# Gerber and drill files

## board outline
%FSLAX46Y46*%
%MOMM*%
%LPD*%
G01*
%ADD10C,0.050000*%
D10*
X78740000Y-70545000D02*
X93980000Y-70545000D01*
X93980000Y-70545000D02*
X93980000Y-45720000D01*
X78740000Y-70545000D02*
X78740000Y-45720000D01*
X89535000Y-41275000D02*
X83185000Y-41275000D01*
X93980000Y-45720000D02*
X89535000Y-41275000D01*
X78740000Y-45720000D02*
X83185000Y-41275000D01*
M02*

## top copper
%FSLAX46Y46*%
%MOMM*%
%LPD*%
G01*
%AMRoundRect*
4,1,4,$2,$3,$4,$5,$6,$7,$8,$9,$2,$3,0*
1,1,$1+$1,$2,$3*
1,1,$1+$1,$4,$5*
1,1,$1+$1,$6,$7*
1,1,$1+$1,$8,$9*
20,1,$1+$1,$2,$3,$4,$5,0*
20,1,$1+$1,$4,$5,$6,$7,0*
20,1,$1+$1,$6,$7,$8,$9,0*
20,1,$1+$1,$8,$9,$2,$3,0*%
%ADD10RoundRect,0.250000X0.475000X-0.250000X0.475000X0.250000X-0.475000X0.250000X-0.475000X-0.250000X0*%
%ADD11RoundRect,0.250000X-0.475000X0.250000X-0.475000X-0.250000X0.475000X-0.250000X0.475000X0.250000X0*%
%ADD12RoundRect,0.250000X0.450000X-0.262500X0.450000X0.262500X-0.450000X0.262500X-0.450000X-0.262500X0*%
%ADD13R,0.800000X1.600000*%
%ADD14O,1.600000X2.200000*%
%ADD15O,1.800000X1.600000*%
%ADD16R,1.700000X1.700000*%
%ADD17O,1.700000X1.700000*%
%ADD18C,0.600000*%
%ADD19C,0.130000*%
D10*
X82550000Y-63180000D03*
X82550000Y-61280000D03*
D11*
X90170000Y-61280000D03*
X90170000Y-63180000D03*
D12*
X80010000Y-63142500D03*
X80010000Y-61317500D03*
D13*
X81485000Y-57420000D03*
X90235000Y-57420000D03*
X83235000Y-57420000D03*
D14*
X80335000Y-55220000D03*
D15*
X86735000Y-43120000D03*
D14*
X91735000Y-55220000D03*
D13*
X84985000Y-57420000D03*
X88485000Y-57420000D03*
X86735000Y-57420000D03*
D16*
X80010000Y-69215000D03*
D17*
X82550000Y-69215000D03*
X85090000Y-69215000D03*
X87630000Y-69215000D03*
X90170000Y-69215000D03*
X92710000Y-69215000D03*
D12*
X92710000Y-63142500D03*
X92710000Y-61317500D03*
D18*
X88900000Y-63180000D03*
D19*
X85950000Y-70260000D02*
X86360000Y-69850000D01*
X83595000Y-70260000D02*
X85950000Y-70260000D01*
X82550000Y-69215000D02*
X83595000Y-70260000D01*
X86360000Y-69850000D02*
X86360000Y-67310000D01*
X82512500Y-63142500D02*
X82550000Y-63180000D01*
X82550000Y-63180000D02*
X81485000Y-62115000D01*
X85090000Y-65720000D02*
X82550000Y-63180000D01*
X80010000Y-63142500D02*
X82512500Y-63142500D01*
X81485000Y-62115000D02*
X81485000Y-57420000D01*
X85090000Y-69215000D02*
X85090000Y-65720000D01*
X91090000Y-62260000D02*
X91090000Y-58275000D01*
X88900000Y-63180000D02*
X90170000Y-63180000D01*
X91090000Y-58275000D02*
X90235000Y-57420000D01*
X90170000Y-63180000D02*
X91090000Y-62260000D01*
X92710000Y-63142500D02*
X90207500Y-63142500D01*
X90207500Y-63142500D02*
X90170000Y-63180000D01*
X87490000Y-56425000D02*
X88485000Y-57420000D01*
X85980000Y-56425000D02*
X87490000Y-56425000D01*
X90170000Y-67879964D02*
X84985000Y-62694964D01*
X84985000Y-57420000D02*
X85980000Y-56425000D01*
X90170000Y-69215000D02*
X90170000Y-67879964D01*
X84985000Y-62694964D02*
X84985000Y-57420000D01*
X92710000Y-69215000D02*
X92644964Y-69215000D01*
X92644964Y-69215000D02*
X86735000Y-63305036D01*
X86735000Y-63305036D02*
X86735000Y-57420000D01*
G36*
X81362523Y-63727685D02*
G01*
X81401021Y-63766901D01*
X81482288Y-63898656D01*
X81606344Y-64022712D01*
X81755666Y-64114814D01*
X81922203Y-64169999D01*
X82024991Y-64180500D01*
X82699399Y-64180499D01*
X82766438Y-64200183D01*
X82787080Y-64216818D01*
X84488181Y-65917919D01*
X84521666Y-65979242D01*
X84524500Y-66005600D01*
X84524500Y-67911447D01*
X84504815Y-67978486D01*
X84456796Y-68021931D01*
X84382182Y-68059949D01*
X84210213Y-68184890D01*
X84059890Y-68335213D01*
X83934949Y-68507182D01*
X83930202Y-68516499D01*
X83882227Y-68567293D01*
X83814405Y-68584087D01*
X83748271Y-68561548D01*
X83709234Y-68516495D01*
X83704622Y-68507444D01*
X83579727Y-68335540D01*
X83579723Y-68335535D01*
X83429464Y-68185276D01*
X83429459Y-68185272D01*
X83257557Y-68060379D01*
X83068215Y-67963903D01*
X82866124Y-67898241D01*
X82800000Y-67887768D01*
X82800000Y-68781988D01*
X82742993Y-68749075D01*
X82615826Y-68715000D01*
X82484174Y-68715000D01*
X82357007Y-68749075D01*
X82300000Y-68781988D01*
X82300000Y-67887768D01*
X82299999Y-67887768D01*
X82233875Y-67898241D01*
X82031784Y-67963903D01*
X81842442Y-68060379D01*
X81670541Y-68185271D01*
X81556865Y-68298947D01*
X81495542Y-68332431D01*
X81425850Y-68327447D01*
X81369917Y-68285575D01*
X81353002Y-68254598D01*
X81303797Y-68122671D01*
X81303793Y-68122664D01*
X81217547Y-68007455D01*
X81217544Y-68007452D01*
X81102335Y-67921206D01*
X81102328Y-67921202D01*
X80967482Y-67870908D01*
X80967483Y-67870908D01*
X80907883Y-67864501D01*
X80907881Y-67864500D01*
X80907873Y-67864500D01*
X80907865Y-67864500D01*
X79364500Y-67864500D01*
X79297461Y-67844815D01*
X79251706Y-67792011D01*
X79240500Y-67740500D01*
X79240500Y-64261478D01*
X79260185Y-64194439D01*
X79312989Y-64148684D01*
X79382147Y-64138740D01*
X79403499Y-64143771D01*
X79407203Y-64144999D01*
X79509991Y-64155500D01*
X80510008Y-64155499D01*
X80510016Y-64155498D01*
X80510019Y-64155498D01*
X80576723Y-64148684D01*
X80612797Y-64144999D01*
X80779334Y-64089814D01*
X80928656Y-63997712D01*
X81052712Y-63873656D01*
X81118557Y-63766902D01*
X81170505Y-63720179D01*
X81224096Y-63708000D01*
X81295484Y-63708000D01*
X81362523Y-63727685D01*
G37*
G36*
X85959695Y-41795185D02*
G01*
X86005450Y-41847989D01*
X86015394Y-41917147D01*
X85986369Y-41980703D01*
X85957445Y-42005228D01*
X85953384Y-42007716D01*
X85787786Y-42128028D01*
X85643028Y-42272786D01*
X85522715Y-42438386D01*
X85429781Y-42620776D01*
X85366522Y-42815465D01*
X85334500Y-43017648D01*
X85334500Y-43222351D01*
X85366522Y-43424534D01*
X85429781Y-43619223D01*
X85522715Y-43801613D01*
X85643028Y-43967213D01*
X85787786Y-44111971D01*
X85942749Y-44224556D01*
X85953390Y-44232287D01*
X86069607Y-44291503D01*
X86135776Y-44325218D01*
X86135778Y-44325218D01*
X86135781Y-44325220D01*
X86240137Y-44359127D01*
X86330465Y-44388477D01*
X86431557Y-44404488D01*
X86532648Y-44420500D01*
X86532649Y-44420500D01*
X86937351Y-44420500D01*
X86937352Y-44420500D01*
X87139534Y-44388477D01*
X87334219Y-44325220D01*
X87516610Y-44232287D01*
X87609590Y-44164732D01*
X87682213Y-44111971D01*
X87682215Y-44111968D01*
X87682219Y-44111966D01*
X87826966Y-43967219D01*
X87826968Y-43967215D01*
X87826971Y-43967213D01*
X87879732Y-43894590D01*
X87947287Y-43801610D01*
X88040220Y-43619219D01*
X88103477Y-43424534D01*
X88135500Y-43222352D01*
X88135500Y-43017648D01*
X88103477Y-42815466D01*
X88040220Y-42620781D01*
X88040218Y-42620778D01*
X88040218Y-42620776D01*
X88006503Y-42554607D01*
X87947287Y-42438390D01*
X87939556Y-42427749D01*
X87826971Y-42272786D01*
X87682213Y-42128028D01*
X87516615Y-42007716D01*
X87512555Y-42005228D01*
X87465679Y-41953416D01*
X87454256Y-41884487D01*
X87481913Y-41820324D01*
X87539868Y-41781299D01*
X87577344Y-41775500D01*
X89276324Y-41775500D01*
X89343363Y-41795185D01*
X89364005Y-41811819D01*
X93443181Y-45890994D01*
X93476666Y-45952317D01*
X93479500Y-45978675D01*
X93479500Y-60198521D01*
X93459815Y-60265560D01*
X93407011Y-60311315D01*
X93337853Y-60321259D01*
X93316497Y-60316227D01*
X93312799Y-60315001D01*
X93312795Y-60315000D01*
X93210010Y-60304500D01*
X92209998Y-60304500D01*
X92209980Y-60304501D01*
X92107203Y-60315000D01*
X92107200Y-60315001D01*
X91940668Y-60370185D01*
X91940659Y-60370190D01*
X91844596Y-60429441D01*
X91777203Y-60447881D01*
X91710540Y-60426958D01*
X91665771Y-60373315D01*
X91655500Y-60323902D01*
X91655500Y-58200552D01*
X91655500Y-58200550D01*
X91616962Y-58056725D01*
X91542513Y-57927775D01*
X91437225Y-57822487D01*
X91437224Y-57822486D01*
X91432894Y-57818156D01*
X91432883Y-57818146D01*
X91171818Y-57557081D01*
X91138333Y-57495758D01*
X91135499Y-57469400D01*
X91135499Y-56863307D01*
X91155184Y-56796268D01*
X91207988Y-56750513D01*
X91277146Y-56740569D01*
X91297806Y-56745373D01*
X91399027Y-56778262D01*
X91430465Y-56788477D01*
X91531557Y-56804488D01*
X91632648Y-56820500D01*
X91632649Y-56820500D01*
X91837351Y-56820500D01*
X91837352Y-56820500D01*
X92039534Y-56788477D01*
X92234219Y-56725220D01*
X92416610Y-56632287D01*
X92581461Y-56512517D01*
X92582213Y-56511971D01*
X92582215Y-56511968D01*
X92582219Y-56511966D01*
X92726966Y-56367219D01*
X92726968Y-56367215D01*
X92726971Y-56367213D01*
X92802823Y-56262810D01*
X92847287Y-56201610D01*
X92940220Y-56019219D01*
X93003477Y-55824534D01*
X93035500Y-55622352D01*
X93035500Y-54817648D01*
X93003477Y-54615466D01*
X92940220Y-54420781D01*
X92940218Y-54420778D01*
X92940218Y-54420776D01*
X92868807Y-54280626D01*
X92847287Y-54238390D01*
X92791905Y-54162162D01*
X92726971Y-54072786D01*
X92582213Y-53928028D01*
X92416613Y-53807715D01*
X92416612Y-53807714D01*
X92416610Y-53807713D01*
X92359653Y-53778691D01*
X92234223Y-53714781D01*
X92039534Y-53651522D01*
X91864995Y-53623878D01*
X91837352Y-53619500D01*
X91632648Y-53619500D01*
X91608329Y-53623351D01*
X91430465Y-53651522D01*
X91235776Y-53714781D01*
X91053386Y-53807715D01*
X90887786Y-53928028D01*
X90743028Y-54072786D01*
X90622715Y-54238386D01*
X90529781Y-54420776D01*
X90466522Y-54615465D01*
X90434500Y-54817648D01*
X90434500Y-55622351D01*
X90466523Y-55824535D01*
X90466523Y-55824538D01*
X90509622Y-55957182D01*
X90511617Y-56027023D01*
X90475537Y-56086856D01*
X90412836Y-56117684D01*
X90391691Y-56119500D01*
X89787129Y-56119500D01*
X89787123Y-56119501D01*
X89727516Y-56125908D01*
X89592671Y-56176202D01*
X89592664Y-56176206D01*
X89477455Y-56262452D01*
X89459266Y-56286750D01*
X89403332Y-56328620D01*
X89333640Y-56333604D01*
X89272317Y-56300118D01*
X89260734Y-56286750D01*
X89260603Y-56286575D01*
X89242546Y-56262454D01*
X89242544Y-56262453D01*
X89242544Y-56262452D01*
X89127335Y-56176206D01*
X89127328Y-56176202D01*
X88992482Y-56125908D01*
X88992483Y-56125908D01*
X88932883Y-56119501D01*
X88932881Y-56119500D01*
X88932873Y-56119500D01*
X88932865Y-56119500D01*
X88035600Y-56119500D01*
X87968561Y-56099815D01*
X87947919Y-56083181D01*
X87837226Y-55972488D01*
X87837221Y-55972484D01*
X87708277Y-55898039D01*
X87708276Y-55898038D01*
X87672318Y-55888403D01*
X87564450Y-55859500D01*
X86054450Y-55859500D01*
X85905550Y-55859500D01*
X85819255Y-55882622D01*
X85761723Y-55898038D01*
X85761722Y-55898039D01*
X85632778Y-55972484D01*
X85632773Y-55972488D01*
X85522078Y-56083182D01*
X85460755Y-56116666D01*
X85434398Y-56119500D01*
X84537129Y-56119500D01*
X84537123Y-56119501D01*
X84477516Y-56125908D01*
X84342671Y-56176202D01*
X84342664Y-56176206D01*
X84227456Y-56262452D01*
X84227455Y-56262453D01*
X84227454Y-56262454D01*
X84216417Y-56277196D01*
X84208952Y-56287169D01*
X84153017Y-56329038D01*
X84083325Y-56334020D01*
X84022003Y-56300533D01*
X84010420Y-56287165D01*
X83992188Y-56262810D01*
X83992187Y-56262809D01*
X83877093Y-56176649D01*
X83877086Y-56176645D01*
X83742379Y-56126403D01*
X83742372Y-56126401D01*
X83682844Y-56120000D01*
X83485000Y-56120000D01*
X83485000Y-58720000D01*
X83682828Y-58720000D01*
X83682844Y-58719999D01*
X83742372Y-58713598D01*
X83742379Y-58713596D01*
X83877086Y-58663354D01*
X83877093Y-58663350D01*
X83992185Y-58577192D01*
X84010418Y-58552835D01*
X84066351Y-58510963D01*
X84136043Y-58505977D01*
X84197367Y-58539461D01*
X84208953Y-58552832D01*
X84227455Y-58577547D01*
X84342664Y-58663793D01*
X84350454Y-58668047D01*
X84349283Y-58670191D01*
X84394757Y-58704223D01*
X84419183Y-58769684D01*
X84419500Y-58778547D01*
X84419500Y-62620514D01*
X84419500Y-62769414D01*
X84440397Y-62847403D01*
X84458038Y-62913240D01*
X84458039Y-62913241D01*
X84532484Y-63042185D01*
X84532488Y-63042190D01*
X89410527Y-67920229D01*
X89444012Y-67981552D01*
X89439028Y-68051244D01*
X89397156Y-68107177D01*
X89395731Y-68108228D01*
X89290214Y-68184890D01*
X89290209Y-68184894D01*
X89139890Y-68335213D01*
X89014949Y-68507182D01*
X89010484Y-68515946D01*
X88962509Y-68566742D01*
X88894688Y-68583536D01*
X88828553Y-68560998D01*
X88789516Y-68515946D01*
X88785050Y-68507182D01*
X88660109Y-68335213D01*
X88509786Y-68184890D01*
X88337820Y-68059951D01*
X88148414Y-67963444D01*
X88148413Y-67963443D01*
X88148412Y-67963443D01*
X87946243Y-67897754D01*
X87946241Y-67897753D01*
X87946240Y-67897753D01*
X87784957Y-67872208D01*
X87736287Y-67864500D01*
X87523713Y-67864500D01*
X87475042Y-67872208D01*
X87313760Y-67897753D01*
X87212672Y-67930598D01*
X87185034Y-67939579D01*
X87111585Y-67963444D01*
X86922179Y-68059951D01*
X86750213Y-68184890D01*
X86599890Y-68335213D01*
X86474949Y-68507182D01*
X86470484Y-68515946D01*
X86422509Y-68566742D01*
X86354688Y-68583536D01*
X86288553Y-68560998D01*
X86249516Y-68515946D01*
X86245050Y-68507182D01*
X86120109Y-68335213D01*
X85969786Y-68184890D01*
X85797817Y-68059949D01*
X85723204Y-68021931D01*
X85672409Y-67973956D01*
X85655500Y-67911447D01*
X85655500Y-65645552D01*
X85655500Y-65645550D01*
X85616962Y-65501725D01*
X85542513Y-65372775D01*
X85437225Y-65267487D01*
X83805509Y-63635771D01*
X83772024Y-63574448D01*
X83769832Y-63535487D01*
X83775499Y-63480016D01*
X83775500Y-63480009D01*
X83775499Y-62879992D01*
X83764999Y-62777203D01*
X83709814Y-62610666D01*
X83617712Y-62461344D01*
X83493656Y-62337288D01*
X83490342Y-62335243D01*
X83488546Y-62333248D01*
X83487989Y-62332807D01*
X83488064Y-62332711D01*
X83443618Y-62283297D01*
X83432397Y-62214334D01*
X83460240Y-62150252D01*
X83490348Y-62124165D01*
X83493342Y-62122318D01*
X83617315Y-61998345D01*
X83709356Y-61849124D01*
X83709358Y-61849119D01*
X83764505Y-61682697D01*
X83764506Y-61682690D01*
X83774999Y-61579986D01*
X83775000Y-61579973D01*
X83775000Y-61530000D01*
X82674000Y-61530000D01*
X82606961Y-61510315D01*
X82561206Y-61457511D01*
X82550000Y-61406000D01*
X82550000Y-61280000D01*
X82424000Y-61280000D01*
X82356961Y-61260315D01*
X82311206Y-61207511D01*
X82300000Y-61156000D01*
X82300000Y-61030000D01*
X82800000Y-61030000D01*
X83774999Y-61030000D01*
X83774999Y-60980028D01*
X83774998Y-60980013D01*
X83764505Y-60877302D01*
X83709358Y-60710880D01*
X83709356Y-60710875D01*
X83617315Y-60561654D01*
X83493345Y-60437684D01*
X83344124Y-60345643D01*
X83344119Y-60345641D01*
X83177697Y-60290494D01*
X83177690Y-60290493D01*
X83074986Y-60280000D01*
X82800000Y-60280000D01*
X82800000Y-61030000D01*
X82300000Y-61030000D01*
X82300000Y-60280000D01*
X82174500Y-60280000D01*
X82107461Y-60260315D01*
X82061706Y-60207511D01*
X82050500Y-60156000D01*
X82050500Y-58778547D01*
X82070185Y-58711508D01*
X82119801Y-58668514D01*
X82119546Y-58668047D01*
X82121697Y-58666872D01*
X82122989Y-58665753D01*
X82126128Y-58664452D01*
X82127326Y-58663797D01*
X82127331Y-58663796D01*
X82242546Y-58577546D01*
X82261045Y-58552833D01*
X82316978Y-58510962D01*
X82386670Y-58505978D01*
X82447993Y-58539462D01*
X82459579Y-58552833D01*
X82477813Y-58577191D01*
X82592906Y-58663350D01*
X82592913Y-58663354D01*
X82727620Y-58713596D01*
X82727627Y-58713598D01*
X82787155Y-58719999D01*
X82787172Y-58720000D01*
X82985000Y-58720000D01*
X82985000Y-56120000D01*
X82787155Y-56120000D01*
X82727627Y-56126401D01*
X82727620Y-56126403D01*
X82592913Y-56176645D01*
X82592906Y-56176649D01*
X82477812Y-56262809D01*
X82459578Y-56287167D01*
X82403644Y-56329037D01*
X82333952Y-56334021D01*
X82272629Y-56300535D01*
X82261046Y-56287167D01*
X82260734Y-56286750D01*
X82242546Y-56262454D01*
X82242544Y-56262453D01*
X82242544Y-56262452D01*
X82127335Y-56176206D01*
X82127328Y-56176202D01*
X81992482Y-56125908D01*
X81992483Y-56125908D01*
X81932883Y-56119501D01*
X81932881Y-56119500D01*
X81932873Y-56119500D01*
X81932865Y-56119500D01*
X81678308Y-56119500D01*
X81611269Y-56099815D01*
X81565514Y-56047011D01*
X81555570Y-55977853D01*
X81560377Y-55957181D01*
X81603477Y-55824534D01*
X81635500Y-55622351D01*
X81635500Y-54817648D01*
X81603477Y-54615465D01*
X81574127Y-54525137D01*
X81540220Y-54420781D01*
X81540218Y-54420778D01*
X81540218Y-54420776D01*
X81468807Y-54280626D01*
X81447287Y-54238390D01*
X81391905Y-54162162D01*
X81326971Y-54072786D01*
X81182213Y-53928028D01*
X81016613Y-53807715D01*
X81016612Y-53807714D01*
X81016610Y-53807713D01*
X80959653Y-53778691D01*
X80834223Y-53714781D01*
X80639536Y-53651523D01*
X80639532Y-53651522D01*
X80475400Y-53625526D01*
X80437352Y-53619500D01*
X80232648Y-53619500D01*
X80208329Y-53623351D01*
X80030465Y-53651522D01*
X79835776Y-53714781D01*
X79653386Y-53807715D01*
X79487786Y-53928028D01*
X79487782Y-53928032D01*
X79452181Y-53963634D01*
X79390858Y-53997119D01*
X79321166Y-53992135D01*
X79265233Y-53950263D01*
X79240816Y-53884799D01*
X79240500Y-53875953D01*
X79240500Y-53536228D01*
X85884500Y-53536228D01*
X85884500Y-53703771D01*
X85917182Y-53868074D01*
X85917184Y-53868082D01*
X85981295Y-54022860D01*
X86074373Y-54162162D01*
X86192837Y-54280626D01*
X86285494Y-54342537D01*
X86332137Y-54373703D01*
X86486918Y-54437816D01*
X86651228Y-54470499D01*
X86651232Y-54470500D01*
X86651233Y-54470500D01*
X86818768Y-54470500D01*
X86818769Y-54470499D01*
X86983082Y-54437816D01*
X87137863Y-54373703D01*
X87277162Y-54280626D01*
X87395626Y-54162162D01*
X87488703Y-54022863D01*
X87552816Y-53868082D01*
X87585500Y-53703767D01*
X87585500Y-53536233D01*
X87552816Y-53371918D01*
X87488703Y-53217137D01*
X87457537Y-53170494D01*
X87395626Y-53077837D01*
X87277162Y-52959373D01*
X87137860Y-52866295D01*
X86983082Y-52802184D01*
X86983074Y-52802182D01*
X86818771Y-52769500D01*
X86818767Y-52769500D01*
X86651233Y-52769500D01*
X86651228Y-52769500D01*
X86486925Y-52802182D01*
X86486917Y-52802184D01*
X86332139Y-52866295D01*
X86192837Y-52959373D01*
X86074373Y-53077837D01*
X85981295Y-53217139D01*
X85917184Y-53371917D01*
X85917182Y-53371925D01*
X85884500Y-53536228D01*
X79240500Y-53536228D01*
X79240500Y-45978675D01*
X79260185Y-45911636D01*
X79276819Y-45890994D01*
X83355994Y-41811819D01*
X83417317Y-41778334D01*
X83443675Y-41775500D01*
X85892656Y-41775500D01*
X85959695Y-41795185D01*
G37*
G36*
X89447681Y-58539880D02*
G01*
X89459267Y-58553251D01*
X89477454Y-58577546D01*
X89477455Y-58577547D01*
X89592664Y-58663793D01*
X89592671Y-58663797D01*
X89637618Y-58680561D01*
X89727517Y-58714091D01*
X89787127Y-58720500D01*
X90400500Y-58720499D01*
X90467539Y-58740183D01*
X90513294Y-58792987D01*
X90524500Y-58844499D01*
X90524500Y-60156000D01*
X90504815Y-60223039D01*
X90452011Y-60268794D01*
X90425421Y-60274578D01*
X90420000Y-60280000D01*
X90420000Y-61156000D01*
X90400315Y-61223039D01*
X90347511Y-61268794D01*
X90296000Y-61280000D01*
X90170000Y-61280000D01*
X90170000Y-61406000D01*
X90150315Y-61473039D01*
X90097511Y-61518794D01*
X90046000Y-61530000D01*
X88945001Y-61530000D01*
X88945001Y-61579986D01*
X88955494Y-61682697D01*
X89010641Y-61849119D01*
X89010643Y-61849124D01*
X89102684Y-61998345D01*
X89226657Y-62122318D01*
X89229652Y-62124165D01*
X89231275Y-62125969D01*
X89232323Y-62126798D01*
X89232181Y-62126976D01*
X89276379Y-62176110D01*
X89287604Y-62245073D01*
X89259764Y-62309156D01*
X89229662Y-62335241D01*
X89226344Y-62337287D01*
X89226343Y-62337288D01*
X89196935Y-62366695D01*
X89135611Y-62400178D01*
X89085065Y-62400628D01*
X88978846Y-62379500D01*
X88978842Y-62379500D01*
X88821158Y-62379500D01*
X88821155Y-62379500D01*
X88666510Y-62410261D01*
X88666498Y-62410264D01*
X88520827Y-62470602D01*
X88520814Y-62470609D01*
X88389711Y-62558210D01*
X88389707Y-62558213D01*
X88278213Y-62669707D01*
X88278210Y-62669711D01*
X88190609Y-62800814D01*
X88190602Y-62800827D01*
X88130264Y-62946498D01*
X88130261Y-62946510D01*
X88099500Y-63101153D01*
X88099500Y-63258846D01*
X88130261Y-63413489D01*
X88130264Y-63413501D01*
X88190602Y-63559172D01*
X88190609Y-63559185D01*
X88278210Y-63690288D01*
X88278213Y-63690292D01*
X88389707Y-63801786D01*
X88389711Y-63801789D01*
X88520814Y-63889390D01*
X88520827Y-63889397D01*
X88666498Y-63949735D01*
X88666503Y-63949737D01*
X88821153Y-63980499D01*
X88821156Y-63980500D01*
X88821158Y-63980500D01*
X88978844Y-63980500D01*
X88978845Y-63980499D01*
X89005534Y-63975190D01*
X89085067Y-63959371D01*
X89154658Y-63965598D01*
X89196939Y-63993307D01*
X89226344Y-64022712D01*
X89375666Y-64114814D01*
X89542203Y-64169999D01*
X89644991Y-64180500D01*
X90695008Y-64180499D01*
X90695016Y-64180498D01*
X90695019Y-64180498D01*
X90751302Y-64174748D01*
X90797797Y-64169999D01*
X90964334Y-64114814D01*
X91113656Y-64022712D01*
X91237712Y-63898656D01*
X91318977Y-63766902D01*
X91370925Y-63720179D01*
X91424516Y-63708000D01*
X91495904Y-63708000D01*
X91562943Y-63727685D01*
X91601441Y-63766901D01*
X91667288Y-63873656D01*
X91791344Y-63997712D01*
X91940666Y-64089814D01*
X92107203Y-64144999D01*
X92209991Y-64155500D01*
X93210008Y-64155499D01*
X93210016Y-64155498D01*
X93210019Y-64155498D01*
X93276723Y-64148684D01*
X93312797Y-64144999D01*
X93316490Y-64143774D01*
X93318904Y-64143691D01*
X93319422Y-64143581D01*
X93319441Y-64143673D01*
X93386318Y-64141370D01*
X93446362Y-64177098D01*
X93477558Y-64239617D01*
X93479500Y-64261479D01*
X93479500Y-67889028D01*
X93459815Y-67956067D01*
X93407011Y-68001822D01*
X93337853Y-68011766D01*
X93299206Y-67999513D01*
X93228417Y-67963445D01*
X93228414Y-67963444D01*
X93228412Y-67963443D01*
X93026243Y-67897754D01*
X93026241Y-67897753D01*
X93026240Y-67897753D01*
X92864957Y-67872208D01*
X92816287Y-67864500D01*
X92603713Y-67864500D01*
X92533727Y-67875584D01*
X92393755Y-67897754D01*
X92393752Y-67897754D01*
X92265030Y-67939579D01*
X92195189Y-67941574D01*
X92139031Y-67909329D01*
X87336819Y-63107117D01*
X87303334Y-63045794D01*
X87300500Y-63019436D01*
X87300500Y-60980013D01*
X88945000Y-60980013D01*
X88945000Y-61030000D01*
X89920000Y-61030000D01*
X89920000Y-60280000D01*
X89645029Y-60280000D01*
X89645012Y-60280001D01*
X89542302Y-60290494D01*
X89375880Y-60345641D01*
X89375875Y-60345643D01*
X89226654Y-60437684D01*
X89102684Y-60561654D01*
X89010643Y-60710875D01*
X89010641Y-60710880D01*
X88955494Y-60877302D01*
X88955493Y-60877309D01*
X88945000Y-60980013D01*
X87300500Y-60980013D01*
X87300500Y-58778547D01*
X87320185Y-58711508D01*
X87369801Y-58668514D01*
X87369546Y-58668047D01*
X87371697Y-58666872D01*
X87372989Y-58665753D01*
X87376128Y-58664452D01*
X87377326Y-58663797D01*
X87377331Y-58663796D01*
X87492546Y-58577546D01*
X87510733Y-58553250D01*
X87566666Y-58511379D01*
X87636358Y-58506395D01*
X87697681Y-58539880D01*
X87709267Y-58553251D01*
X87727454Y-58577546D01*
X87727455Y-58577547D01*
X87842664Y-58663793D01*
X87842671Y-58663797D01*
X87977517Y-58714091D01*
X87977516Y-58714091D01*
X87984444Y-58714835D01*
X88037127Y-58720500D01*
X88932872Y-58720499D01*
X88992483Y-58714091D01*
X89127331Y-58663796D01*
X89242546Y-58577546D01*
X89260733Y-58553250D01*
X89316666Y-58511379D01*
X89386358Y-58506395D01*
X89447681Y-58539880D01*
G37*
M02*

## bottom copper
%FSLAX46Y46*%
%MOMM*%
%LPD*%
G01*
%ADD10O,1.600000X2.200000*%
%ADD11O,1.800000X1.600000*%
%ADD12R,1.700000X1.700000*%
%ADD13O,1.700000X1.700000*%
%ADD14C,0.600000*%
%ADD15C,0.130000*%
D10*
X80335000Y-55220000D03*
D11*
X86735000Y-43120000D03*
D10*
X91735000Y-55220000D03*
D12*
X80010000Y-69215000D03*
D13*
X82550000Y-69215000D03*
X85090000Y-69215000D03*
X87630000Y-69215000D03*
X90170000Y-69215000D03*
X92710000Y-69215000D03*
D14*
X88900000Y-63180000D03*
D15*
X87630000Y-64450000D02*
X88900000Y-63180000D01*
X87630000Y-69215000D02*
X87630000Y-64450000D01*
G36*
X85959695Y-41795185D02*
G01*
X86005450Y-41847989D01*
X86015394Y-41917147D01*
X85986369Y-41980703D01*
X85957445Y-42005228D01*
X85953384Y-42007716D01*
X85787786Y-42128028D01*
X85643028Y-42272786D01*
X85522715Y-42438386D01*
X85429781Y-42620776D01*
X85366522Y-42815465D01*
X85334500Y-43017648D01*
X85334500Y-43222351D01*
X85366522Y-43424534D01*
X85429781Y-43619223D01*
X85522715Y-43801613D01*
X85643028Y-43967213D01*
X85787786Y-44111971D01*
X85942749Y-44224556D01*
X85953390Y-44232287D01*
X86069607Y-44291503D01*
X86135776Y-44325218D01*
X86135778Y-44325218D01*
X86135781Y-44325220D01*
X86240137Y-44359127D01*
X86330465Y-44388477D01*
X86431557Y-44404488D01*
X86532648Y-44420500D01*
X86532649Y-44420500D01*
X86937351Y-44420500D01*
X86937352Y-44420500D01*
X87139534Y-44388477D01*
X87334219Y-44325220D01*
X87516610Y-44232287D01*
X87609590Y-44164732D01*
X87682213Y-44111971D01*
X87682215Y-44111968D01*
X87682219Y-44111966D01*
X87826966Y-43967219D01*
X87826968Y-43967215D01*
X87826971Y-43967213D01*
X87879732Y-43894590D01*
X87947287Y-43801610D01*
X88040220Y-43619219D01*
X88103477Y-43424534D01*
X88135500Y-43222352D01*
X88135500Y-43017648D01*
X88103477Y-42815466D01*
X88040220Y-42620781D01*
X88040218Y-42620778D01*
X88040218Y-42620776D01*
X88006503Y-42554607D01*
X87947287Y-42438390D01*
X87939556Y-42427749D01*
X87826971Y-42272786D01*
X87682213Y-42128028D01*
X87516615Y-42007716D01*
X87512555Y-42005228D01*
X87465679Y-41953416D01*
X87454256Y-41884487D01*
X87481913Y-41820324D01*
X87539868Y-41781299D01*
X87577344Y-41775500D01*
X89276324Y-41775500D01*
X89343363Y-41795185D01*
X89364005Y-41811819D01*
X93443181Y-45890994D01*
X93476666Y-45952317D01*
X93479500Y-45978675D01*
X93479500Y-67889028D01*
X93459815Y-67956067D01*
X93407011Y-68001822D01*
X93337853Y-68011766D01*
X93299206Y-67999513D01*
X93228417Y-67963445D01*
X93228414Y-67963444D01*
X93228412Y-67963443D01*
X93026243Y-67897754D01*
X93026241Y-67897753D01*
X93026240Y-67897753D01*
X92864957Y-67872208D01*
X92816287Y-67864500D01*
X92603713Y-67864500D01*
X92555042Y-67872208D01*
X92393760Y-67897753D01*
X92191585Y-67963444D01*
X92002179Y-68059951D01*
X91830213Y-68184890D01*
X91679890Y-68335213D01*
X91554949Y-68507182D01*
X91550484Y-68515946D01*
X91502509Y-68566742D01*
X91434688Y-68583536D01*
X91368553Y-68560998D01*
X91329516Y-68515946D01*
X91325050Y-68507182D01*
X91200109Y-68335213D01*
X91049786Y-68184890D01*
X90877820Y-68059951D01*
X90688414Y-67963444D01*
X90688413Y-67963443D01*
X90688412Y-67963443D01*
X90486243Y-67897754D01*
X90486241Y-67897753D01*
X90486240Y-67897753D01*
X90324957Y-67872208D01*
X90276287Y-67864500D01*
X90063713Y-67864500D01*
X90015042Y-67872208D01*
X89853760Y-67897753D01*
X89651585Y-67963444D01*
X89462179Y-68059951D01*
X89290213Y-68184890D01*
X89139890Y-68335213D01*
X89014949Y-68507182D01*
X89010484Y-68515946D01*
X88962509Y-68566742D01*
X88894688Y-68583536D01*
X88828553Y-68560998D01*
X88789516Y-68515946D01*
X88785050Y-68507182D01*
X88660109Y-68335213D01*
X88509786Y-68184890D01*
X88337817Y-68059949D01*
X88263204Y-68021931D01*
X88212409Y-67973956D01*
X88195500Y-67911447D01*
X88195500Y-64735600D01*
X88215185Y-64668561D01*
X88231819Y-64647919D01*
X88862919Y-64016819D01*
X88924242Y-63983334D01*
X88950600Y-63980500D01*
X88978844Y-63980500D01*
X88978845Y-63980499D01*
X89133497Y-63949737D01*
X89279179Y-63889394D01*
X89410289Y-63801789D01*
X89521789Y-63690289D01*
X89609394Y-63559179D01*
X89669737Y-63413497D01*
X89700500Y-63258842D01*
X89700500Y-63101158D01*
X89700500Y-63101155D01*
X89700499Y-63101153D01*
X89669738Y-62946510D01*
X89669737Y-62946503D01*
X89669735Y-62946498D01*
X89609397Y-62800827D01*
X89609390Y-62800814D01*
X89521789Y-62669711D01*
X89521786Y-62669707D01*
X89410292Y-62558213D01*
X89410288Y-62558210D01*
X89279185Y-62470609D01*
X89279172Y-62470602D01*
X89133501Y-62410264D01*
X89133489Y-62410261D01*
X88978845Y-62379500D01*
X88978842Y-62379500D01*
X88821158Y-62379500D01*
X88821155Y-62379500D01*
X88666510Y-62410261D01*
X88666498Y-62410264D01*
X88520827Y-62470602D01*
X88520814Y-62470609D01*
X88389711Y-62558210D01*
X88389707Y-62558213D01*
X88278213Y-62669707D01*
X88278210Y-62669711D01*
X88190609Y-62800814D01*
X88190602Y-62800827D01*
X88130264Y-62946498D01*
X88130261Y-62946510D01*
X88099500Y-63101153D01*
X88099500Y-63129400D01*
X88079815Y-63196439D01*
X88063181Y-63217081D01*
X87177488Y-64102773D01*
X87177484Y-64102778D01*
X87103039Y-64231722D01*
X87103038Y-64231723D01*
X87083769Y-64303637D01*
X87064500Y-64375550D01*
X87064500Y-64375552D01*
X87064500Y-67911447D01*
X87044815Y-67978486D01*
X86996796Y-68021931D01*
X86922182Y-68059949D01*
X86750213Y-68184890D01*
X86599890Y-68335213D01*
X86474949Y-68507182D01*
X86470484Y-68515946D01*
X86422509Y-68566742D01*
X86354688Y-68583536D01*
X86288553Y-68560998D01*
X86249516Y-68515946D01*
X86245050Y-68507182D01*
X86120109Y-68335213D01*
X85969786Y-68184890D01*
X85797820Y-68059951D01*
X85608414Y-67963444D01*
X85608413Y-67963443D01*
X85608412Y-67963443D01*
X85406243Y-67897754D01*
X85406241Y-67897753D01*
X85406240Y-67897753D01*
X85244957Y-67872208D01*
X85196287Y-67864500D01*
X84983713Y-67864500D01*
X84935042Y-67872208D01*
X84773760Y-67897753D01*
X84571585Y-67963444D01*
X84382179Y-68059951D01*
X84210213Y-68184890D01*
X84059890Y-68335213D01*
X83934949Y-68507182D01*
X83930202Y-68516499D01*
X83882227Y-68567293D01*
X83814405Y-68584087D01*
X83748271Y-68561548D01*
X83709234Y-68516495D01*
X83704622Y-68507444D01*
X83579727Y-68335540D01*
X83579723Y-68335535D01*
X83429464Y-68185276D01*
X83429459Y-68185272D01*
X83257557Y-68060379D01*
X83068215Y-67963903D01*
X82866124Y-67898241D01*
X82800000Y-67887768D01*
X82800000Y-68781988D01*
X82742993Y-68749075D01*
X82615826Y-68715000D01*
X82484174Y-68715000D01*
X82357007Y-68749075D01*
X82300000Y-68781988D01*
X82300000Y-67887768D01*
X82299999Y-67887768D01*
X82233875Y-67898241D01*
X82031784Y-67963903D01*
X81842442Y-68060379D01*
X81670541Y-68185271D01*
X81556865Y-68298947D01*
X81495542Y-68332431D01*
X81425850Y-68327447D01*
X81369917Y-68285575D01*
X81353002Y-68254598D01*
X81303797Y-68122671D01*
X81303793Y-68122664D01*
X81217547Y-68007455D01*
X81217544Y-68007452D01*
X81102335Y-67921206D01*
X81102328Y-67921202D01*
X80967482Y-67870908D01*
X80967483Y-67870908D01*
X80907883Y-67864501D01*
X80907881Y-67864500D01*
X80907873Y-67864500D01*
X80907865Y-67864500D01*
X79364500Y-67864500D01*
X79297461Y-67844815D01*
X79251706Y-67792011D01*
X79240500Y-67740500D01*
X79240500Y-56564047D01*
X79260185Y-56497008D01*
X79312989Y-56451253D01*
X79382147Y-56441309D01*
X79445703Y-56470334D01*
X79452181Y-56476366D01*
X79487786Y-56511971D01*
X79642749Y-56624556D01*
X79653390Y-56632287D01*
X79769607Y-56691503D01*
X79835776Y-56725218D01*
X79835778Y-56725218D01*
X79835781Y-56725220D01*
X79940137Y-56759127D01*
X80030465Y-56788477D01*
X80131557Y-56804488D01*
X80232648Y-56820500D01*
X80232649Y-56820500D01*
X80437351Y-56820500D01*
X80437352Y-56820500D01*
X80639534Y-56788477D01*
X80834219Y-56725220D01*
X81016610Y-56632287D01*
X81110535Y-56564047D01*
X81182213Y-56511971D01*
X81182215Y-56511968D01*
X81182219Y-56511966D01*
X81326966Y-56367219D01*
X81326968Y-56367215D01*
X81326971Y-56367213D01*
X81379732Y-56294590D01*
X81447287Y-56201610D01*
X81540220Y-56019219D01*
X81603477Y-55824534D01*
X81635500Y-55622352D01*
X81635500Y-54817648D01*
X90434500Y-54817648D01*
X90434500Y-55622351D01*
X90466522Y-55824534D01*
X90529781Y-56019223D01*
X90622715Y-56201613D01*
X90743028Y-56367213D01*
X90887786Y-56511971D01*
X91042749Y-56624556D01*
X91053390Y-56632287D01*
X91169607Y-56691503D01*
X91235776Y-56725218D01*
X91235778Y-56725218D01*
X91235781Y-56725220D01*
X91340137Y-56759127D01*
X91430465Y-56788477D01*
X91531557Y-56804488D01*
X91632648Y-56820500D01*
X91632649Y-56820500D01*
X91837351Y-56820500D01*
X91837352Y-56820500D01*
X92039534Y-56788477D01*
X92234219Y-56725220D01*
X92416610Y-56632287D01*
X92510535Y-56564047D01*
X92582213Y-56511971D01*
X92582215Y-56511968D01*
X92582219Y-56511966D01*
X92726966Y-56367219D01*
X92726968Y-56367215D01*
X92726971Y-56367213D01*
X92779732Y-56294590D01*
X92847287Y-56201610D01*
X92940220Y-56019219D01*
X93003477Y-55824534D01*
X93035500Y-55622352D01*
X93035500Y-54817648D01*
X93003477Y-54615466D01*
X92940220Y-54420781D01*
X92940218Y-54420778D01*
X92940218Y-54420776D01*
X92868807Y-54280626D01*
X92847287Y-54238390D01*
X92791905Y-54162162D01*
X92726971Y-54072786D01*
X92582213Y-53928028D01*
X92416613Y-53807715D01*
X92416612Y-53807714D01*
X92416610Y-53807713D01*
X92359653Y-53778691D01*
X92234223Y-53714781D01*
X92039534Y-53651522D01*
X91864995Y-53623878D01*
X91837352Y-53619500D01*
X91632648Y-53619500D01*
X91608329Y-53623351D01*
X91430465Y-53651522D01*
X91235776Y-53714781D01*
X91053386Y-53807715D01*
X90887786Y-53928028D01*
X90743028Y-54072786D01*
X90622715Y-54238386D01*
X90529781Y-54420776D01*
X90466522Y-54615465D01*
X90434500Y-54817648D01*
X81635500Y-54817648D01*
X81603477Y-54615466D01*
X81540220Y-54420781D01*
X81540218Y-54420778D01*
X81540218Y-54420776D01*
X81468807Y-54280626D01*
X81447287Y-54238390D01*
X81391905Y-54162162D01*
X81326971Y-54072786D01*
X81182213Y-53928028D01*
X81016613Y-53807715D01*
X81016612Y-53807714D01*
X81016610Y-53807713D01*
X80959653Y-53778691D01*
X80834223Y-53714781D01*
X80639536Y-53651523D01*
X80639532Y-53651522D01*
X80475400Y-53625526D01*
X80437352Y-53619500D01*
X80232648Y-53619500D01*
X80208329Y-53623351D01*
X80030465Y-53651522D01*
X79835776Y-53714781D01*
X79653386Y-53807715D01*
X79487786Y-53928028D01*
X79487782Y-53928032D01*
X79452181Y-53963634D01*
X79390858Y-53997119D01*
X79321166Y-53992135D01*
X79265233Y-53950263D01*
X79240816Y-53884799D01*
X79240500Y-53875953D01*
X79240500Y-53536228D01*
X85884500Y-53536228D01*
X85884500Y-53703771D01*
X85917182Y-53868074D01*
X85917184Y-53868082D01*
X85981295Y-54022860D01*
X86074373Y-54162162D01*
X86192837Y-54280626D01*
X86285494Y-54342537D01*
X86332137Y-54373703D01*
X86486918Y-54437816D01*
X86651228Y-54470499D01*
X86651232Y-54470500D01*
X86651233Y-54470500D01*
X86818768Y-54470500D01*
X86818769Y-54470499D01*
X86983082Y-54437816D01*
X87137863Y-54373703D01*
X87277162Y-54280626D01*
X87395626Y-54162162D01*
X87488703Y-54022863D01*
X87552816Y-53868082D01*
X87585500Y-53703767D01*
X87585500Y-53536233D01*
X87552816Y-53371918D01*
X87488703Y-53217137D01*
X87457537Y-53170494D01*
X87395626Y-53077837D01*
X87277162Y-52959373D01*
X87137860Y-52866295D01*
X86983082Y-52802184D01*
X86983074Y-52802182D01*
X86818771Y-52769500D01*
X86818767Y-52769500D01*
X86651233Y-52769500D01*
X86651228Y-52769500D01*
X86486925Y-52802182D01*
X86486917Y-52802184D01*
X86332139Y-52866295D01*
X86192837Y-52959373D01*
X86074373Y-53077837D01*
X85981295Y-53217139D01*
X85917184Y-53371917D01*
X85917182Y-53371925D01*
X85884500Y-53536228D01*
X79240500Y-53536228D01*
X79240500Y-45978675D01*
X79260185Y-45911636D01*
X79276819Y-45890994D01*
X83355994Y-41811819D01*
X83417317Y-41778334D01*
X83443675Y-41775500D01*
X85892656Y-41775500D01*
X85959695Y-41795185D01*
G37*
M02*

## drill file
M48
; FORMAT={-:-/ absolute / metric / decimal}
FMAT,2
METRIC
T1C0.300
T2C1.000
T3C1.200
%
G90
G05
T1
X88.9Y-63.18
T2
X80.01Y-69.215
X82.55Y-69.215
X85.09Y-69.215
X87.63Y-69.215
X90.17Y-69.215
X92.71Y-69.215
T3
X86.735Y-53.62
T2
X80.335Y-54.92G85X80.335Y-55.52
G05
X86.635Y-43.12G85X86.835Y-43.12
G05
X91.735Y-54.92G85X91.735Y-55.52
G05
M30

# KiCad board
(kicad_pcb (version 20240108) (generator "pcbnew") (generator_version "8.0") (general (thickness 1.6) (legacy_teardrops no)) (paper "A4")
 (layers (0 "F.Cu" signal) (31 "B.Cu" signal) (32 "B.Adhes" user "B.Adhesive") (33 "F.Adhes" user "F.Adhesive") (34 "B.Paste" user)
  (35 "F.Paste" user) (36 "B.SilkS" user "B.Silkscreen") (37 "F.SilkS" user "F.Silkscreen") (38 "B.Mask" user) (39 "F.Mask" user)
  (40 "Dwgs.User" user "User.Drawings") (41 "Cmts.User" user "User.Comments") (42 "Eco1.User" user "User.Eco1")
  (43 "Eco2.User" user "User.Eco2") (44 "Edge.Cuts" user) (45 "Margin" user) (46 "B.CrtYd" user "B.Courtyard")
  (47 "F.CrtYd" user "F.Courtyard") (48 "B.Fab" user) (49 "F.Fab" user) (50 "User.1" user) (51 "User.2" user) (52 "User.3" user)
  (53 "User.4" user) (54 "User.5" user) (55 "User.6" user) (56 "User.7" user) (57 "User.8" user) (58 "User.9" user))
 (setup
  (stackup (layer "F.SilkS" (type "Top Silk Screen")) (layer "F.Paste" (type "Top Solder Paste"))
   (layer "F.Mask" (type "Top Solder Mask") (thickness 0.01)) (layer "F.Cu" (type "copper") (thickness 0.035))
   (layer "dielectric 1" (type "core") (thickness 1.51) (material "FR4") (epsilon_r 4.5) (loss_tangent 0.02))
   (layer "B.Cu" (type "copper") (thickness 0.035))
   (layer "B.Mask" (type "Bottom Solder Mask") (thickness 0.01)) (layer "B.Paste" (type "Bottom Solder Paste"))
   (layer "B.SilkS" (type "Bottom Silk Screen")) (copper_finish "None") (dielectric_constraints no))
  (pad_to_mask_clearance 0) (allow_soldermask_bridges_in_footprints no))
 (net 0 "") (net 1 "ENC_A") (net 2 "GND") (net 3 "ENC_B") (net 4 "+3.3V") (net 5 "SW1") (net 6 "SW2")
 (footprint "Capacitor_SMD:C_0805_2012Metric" (layer "F.Cu") (at 82.55 62.23 90)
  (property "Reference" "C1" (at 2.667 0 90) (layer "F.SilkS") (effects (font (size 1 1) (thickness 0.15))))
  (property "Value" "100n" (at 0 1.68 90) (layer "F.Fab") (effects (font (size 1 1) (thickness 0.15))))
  (pad "1" smd roundrect (at -0.95 0 90) (size 1 1.45) (layers "F.Cu" "F.Paste" "F.Mask") (roundrect_rratio 0.25) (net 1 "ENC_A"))
  (pad "2" smd roundrect (at 0.95 0 90) (size 1 1.45) (layers "F.Cu" "F.Paste" "F.Mask") (roundrect_rratio 0.25) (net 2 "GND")))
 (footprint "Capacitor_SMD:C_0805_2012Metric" (layer "F.Cu") (at 90.17 62.23 -90)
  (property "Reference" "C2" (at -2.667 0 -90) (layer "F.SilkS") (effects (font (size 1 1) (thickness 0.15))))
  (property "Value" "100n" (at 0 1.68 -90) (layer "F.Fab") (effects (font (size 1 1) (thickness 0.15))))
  (pad "1" smd roundrect (at -0.95 0 270) (size 1 1.45) (layers "F.Cu" "F.Paste" "F.Mask") (roundrect_rratio 0.25) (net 2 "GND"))
  (pad "2" smd roundrect (at 0.95 0 270) (size 1 1.45) (layers "F.Cu" "F.Paste" "F.Mask") (roundrect_rratio 0.25) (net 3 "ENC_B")))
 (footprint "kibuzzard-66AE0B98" (layer "F.Cu") (at 85.09 65.786 90)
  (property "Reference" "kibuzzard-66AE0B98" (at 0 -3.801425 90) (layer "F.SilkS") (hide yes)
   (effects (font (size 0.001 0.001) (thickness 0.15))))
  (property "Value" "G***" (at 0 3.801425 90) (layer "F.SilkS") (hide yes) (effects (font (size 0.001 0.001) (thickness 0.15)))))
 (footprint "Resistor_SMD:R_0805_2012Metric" (layer "F.Cu") (at 80.01 62.23 90)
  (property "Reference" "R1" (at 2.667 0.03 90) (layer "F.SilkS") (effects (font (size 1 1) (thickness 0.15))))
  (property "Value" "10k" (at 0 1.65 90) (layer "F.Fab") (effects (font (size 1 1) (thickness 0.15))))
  (pad "1" smd roundrect (at -0.9125 0 90) (size 1.025 1.4) (layers "F.Cu" "F.Paste" "F.Mask") (roundrect_rratio 0.243902) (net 1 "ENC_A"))
  (pad "2" smd roundrect (at 0.9125 0 90) (size 1.025 1.4) (layers "F.Cu" "F.Paste" "F.Mask") (roundrect_rratio 0.243902) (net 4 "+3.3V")))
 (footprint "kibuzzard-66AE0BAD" (layer "F.Cu") (at 90.17 66.288192 90)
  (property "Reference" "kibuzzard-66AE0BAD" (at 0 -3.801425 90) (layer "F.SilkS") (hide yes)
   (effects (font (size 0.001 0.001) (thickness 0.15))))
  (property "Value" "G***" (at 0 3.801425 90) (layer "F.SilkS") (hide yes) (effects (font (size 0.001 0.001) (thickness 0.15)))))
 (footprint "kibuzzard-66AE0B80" (layer "F.Cu") (at 82.55 66.174767 90)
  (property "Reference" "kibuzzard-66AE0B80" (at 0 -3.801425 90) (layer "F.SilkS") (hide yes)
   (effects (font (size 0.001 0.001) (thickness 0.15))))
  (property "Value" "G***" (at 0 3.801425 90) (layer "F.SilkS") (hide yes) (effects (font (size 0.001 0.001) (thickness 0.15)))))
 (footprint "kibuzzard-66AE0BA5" (layer "F.Cu") (at 87.63 65.806548 90)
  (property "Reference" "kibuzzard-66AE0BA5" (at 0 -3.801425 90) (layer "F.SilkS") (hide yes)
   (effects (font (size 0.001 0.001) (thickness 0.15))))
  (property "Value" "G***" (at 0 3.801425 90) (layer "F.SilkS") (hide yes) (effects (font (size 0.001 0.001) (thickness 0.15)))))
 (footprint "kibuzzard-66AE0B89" (layer "F.Cu") (at 80.01 66.198603 90)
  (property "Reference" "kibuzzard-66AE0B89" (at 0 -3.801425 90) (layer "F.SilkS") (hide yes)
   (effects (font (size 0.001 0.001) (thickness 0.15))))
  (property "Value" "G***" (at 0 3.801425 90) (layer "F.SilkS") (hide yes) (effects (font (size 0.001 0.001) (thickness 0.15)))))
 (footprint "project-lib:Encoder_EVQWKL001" (layer "F.Cu") (at 86.735 53.62)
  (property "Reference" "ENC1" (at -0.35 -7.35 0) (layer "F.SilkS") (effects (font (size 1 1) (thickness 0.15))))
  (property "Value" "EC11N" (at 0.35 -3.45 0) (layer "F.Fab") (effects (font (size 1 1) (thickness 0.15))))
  (pad "" np_thru_hole circle (at 0 0) (size 1.2 1.2) (drill 1.2) (layers "F&B.Cu"))
  (pad "A" smd rect (at -5.25 3.8) (size 0.8 1.6) (layers "F.Cu" "F.Paste" "F.Mask") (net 1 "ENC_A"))
  (pad "B" smd rect (at 3.5 3.8) (size 0.8 1.6) (layers "F.Cu" "F.Paste" "F.Mask") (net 3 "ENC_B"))
  (pad "C" smd rect (at -3.5 3.8) (size 0.8 1.6) (layers "F.Cu" "F.Paste" "F.Mask") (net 2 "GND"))
  (pad "GND" thru_hole oval (at -6.4 1.6) (size 1.6 2.2) (drill oval 1 1.6) (layers "*.Cu" "*.Mask") (remove_unused_layers no))
  (pad "GND" thru_hole oval (at 0 -10.5) (size 1.8 1.6) (drill oval 1.2 1) (layers "*.Cu" "*.Mask") (remove_unused_layers no))
  (pad "GND" thru_hole oval (at 5 1.6) (size 1.6 2.2) (drill oval 1 1.6) (layers "*.Cu" "*.Mask") (remove_unused_layers no))
  (pad "S1" smd rect (at -1.75 3.8) (size 0.8 1.6) (layers "F.Cu" "F.Paste" "F.Mask") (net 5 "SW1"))
  (pad "S1" smd rect (at 1.75 3.8) (size 0.8 1.6) (layers "F.Cu" "F.Paste" "F.Mask") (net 5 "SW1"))
  (pad "S2" smd rect (at 0 3.8) (size 0.8 1.6) (layers "F.Cu" "F.Paste" "F.Mask") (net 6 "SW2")))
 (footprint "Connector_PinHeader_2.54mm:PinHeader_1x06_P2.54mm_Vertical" (layer "F.Cu") (at 80.01 69.215 90)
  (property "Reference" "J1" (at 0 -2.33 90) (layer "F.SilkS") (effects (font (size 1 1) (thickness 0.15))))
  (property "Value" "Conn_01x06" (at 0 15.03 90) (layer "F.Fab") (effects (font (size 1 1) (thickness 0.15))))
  (pad "1" thru_hole rect (at 0 0 90) (size 1.7 1.7) (drill 1) (layers "*.Cu" "*.Mask") (remove_unused_layers no) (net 4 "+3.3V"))
  (pad "2" thru_hole oval (at 0 2.54 90) (size 1.7 1.7) (drill 1) (layers "*.Cu" "*.Mask") (remove_unused_layers no) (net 2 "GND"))
  (pad "3" thru_hole oval (at 0 5.08 90) (size 1.7 1.7) (drill 1) (layers "*.Cu" "*.Mask") (remove_unused_layers no) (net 1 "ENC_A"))
  (pad "4" thru_hole oval (at 0 7.62 90) (size 1.7 1.7) (drill 1) (layers "*.Cu" "*.Mask") (remove_unused_layers no) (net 3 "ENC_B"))
  (pad "5" thru_hole oval (at 0 10.16 90) (size 1.7 1.7) (drill 1) (layers "*.Cu" "*.Mask") (remove_unused_layers no) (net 5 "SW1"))
  (pad "6" thru_hole oval (at 0 12.7 90) (size 1.7 1.7) (drill 1) (layers "*.Cu" "*.Mask") (remove_unused_layers no) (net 6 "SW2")))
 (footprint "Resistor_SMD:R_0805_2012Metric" (layer "F.Cu") (at 92.71 62.23 90)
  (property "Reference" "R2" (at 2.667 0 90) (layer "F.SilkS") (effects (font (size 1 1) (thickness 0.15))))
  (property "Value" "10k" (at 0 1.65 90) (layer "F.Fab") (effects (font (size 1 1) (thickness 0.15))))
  (pad "1" smd roundrect (at -0.9125 0 90) (size 1.025 1.4) (layers "F.Cu" "F.Paste" "F.Mask") (roundrect_rratio 0.243902) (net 3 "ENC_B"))
  (pad "2" smd roundrect (at 0.9125 0 90) (size 1.025 1.4) (layers "F.Cu" "F.Paste" "F.Mask") (roundrect_rratio 0.243902) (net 4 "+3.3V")))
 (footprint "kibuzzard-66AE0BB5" (layer "F.Cu") (at 92.71 66.229836 90)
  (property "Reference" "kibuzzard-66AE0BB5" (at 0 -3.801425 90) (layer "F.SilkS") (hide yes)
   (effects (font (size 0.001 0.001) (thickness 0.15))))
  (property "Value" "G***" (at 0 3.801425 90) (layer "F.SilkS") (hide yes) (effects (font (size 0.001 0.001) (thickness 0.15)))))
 (gr_line (start 78.74 70.545) (end 93.98 70.545) (stroke (width 0.05) (type default)) (layer "Edge.Cuts"))
 (gr_line (start 93.98 70.545) (end 93.98 45.72) (stroke (width 0.05) (type default)) (layer "Edge.Cuts"))
 (gr_line (start 78.74 70.545) (end 78.74 45.72) (stroke (width 0.05) (type default)) (layer "Edge.Cuts"))
 (gr_line (start 89.535 41.275) (end 83.185 41.275) (stroke (width 0.05) (type default)) (layer "Edge.Cuts"))
 (gr_line (start 93.98 45.72) (end 89.535 41.275) (stroke (width 0.05) (type default)) (layer "Edge.Cuts"))
 (gr_line (start 78.74 45.72) (end 83.185 41.275) (stroke (width 0.05) (type default)) (layer "Edge.Cuts"))
 (segment (start 85.95 70.26) (end 86.36 69.85) (width 0.13) (layer "F.Cu") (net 2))
 (segment (start 83.595 70.26) (end 85.95 70.26) (width 0.13) (layer "F.Cu") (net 2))
 (segment (start 82.55 69.215) (end 83.595 70.26) (width 0.13) (layer "F.Cu") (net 2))
 (segment (start 86.36 69.85) (end 86.36 67.31) (width 0.13) (layer "F.Cu") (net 2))
 (segment (start 82.5125 63.1425) (end 82.55 63.18) (width 0.13) (layer "F.Cu") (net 1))
 (segment (start 82.55 63.18) (end 81.485 62.115) (width 0.13) (layer "F.Cu") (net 1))
 (segment (start 85.09 65.72) (end 82.55 63.18) (width 0.13) (layer "F.Cu") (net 1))
 (segment (start 80.01 63.1425) (end 82.5125 63.1425) (width 0.13) (layer "F.Cu") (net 1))
 (segment (start 81.485 62.115) (end 81.485 57.42) (width 0.13) (layer "F.Cu") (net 1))
 (segment (start 85.09 69.215) (end 85.09 65.72) (width 0.13) (layer "F.Cu") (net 1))
 (segment (start 91.09 62.26) (end 91.09 58.275) (width 0.13) (layer "F.Cu") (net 3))
 (segment (start 88.9 63.18) (end 90.17 63.18) (width 0.13) (layer "F.Cu") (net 3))
 (segment (start 91.09 58.275) (end 90.235 57.42) (width 0.13) (layer "F.Cu") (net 3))
 (segment (start 90.17 63.18) (end 91.09 62.26) (width 0.13) (layer "F.Cu") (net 3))
 (segment (start 92.71 63.1425) (end 90.2075 63.1425) (width 0.13) (layer "F.Cu") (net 3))
 (segment (start 90.2075 63.1425) (end 90.17 63.18) (width 0.13) (layer "F.Cu") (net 3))
 (via (at 88.9 63.18) (size 0.6) (drill 0.3) (layers "F.Cu" "B.Cu") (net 3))
 (segment (start 87.63 64.45) (end 88.9 63.18) (width 0.13) (layer "B.Cu") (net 3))
 (segment (start 87.63 69.215) (end 87.63 64.45) (width 0.13) (layer "B.Cu") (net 3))
 (segment (start 87.49 56.425) (end 88.485 57.42) (width 0.13) (layer "F.Cu") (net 5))
 (segment (start 85.98 56.425) (end 87.49 56.425) (width 0.13) (layer "F.Cu") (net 5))
 (segment (start 90.17 67.879964) (end 84.985 62.694964) (width 0.13) (layer "F.Cu") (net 5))
 (segment (start 84.985 57.42) (end 85.98 56.425) (width 0.13) (layer "F.Cu") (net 5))
 (segment (start 90.17 69.215) (end 90.17 67.879964) (width 0.13) (layer "F.Cu") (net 5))
 (segment (start 84.985 62.694964) (end 84.985 57.42) (width 0.13) (layer "F.Cu") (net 5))
 (segment (start 92.71 69.215) (end 92.644964 69.215) (width 0.13) (layer "F.Cu") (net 6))
 (segment (start 92.644964 69.215) (end 86.735 63.305036) (width 0.13) (layer "F.Cu") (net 6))
 (segment (start 86.735 63.305036) (end 86.735 57.42) (width 0.13) (layer "F.Cu") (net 6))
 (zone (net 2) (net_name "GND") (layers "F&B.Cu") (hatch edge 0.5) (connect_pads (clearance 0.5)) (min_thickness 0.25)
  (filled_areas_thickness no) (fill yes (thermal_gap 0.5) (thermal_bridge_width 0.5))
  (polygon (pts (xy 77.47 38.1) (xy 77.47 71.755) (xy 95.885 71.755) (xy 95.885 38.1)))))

